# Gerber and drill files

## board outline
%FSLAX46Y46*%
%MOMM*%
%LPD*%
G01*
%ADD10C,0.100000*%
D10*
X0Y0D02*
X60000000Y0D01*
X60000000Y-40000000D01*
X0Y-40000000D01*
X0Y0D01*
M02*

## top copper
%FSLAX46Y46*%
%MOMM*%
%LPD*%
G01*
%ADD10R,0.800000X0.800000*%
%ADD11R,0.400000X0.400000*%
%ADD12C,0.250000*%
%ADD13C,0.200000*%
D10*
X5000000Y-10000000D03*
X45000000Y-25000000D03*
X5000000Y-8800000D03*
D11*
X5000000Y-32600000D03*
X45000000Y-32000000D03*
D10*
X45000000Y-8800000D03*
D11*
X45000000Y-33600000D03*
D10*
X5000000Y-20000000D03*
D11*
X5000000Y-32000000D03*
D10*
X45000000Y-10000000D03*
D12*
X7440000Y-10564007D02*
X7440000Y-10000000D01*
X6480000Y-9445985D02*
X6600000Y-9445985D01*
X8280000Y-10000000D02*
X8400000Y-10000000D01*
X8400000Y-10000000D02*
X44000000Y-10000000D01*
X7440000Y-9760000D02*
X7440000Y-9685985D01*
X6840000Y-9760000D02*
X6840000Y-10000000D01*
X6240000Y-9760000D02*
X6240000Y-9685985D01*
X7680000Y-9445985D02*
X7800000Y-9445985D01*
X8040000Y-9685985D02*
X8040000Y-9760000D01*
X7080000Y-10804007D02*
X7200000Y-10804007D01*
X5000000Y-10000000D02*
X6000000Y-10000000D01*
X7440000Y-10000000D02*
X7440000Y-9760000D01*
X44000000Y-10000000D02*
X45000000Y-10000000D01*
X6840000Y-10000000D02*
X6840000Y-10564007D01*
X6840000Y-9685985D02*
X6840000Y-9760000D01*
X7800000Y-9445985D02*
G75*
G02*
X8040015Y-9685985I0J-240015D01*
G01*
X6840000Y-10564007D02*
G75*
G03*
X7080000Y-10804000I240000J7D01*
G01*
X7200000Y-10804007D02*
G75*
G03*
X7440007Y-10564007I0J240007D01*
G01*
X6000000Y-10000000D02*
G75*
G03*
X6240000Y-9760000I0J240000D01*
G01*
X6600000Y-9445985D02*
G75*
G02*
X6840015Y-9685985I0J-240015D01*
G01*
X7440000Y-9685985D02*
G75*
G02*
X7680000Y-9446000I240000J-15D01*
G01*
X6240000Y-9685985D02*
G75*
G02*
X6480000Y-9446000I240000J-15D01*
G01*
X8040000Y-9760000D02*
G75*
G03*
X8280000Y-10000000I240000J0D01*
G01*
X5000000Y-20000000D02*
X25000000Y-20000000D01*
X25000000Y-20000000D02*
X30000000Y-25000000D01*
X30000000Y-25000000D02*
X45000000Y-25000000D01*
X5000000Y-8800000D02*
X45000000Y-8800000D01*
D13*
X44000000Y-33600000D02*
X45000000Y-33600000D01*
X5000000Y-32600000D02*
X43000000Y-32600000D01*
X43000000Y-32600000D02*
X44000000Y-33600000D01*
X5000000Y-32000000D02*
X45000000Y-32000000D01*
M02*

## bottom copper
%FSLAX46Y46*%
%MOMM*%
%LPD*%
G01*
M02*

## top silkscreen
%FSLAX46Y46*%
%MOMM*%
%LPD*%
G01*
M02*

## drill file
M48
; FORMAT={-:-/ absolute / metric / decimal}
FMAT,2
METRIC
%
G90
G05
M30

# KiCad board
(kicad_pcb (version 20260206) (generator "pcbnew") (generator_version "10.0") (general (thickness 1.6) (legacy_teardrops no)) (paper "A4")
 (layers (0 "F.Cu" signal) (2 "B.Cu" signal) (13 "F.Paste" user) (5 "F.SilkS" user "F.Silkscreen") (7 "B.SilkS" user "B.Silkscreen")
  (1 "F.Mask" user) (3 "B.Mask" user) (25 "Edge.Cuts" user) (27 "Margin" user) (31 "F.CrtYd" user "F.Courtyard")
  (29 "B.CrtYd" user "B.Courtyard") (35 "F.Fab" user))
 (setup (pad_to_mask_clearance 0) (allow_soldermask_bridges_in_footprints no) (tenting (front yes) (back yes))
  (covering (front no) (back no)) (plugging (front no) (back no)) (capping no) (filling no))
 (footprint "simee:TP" (layer "F.Cu") (at 5 10)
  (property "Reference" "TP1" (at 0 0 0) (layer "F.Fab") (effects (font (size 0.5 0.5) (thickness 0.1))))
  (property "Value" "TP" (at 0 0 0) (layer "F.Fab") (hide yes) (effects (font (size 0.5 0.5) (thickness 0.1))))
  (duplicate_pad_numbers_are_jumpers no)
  (pad "1" smd rect (at 0 0) (size 0.8 0.8) (layers "F.Cu" "F.Mask") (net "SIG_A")))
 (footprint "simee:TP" (layer "F.Cu") (at 45 25)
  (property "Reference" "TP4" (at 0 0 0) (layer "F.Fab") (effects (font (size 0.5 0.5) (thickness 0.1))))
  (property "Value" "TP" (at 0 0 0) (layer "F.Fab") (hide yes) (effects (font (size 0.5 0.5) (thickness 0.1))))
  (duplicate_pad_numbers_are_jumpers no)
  (pad "1" smd rect (at 0 0) (size 0.8 0.8) (layers "F.Cu" "F.Mask") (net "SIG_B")))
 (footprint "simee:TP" (layer "F.Cu") (at 5 8.8)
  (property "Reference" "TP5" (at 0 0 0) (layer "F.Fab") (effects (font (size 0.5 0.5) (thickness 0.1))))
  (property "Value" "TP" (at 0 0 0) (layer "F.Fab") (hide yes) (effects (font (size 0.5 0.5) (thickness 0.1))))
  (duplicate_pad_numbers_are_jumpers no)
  (pad "1" smd rect (at 0 0) (size 0.8 0.8) (layers "F.Cu" "F.Mask") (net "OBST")))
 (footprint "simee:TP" (layer "F.Cu") (at 5 32.6)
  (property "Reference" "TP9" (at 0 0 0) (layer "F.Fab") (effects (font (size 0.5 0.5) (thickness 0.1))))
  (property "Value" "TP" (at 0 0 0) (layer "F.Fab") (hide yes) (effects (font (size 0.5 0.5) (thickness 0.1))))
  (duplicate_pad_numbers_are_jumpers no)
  (pad "1" smd rect (at 0 0) (size 0.4 0.4) (layers "F.Cu" "F.Mask") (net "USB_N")))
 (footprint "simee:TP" (layer "F.Cu") (at 45 32)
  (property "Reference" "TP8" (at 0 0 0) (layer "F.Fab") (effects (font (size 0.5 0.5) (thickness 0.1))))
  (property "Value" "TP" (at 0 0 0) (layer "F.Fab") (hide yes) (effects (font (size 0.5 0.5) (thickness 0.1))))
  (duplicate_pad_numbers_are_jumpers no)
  (pad "1" smd rect (at 0 0) (size 0.4 0.4) (layers "F.Cu" "F.Mask") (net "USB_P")))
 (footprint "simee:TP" (layer "F.Cu") (at 45 8.8)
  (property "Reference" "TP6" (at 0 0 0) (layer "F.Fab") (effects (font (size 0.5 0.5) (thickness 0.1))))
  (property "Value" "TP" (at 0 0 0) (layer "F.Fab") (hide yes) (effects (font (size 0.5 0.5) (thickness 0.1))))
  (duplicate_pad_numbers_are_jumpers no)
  (pad "1" smd rect (at 0 0) (size 0.8 0.8) (layers "F.Cu" "F.Mask") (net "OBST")))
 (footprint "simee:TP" (layer "F.Cu") (at 45 33.6)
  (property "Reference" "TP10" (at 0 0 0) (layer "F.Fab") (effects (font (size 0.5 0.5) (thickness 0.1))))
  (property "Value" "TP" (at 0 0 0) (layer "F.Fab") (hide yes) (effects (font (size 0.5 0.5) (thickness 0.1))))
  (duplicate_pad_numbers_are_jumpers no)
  (pad "1" smd rect (at 0 0) (size 0.4 0.4) (layers "F.Cu" "F.Mask") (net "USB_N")))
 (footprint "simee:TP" (layer "F.Cu") (at 5 20)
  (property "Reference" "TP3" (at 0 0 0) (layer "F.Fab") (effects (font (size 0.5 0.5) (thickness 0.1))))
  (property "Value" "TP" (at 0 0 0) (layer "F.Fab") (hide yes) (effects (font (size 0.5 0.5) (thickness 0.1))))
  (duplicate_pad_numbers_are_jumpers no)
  (pad "1" smd rect (at 0 0) (size 0.8 0.8) (layers "F.Cu" "F.Mask") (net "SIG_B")))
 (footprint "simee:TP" (layer "F.Cu") (at 5 32)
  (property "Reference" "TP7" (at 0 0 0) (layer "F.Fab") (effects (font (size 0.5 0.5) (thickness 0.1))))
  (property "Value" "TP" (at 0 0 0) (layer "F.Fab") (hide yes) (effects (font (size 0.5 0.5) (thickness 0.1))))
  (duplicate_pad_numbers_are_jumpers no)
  (pad "1" smd rect (at 0 0) (size 0.4 0.4) (layers "F.Cu" "F.Mask") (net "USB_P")))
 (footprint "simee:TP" (layer "F.Cu") (at 45 10)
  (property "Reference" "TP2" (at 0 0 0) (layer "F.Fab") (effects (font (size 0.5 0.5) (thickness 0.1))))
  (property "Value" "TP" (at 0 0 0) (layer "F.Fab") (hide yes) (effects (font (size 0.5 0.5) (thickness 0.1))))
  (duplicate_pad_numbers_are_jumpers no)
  (pad "1" smd rect (at 0 0) (size 0.8 0.8) (layers "F.Cu" "F.Mask") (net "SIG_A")))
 (gr_rect (start 0 0) (end 60 40) (stroke (width 0.1) (type default)) (fill no) (layer "Edge.Cuts"))
 (segment (start 7.44 10.564007) (end 7.44 10) (width 0.25) (layer "F.Cu") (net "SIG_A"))
 (segment (start 6.48 9.445985) (end 6.6 9.445985) (width 0.25) (layer "F.Cu") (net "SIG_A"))
 (segment (start 8.28 10) (end 8.4 10) (width 0.25) (layer "F.Cu") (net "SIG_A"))
 (segment (start 8.4 10) (end 44 10) (width 0.25) (layer "F.Cu") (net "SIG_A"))
 (segment (start 7.44 9.76) (end 7.44 9.685985) (width 0.25) (layer "F.Cu") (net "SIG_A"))
 (segment (start 6.84 9.76) (end 6.84 10) (width 0.25) (layer "F.Cu") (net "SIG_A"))
 (segment (start 6.24 9.76) (end 6.24 9.685985) (width 0.25) (layer "F.Cu") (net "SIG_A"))
 (segment (start 7.68 9.445985) (end 7.8 9.445985) (width 0.25) (layer "F.Cu") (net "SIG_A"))
 (segment (start 8.04 9.685985) (end 8.04 9.76) (width 0.25) (layer "F.Cu") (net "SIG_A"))
 (segment (start 7.08 10.804007) (end 7.2 10.804007) (width 0.25) (layer "F.Cu") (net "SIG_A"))
 (segment (start 5 10) (end 6 10) (width 0.25) (layer "F.Cu") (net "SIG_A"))
 (segment (start 7.44 10) (end 7.44 9.76) (width 0.25) (layer "F.Cu") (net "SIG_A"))
 (segment (start 44 10) (end 45 10) (width 0.25) (layer "F.Cu") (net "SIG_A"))
 (segment (start 6.84 10) (end 6.84 10.564007) (width 0.25) (layer "F.Cu") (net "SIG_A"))
 (segment (start 6.84 9.685985) (end 6.84 9.76) (width 0.25) (layer "F.Cu") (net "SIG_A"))
 (arc (start 7.8 9.445985) (mid 7.969706 9.516279) (end 8.04 9.685985) (width 0.25) (layer "F.Cu") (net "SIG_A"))
 (arc (start 6.84 10.564007) (mid 6.910294 10.733713) (end 7.08 10.804007) (width 0.25) (layer "F.Cu") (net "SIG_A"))
 (arc (start 7.2 10.804007) (mid 7.369706 10.733713) (end 7.44 10.564007) (width 0.25) (layer "F.Cu") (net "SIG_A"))
 (arc (start 6 10) (mid 6.169706 9.929706) (end 6.24 9.76) (width 0.25) (layer "F.Cu") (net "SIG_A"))
 (arc (start 6.6 9.445985) (mid 6.769706 9.516279) (end 6.84 9.685985) (width 0.25) (layer "F.Cu") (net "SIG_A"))
 (arc (start 7.44 9.685985) (mid 7.510294 9.516279) (end 7.68 9.445985) (width 0.25) (layer "F.Cu") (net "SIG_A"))
 (arc (start 6.24 9.685985) (mid 6.310294 9.516279) (end 6.48 9.445985) (width 0.25) (layer "F.Cu") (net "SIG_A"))
 (arc (start 8.04 9.76) (mid 8.110294 9.929706) (end 8.28 10) (width 0.25) (layer "F.Cu") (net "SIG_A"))
 (segment (start 5 20) (end 25 20) (width 0.25) (layer "F.Cu") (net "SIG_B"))
 (segment (start 25 20) (end 30 25) (width 0.25) (layer "F.Cu") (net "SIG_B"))
 (segment (start 30 25) (end 45 25) (width 0.25) (layer "F.Cu") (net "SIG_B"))
 (segment (start 5 8.8) (end 45 8.8) (width 0.25) (layer "F.Cu") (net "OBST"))
 (segment (start 44 33.6) (end 45 33.6) (width 0.2) (layer "F.Cu") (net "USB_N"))
 (segment (start 5 32.6) (end 43 32.6) (width 0.2) (layer "F.Cu") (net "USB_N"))
 (segment (start 43 32.6) (end 44 33.6) (width 0.2) (layer "F.Cu") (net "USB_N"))
 (segment (start 5 32) (end 45 32) (width 0.2) (layer "F.Cu") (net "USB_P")))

